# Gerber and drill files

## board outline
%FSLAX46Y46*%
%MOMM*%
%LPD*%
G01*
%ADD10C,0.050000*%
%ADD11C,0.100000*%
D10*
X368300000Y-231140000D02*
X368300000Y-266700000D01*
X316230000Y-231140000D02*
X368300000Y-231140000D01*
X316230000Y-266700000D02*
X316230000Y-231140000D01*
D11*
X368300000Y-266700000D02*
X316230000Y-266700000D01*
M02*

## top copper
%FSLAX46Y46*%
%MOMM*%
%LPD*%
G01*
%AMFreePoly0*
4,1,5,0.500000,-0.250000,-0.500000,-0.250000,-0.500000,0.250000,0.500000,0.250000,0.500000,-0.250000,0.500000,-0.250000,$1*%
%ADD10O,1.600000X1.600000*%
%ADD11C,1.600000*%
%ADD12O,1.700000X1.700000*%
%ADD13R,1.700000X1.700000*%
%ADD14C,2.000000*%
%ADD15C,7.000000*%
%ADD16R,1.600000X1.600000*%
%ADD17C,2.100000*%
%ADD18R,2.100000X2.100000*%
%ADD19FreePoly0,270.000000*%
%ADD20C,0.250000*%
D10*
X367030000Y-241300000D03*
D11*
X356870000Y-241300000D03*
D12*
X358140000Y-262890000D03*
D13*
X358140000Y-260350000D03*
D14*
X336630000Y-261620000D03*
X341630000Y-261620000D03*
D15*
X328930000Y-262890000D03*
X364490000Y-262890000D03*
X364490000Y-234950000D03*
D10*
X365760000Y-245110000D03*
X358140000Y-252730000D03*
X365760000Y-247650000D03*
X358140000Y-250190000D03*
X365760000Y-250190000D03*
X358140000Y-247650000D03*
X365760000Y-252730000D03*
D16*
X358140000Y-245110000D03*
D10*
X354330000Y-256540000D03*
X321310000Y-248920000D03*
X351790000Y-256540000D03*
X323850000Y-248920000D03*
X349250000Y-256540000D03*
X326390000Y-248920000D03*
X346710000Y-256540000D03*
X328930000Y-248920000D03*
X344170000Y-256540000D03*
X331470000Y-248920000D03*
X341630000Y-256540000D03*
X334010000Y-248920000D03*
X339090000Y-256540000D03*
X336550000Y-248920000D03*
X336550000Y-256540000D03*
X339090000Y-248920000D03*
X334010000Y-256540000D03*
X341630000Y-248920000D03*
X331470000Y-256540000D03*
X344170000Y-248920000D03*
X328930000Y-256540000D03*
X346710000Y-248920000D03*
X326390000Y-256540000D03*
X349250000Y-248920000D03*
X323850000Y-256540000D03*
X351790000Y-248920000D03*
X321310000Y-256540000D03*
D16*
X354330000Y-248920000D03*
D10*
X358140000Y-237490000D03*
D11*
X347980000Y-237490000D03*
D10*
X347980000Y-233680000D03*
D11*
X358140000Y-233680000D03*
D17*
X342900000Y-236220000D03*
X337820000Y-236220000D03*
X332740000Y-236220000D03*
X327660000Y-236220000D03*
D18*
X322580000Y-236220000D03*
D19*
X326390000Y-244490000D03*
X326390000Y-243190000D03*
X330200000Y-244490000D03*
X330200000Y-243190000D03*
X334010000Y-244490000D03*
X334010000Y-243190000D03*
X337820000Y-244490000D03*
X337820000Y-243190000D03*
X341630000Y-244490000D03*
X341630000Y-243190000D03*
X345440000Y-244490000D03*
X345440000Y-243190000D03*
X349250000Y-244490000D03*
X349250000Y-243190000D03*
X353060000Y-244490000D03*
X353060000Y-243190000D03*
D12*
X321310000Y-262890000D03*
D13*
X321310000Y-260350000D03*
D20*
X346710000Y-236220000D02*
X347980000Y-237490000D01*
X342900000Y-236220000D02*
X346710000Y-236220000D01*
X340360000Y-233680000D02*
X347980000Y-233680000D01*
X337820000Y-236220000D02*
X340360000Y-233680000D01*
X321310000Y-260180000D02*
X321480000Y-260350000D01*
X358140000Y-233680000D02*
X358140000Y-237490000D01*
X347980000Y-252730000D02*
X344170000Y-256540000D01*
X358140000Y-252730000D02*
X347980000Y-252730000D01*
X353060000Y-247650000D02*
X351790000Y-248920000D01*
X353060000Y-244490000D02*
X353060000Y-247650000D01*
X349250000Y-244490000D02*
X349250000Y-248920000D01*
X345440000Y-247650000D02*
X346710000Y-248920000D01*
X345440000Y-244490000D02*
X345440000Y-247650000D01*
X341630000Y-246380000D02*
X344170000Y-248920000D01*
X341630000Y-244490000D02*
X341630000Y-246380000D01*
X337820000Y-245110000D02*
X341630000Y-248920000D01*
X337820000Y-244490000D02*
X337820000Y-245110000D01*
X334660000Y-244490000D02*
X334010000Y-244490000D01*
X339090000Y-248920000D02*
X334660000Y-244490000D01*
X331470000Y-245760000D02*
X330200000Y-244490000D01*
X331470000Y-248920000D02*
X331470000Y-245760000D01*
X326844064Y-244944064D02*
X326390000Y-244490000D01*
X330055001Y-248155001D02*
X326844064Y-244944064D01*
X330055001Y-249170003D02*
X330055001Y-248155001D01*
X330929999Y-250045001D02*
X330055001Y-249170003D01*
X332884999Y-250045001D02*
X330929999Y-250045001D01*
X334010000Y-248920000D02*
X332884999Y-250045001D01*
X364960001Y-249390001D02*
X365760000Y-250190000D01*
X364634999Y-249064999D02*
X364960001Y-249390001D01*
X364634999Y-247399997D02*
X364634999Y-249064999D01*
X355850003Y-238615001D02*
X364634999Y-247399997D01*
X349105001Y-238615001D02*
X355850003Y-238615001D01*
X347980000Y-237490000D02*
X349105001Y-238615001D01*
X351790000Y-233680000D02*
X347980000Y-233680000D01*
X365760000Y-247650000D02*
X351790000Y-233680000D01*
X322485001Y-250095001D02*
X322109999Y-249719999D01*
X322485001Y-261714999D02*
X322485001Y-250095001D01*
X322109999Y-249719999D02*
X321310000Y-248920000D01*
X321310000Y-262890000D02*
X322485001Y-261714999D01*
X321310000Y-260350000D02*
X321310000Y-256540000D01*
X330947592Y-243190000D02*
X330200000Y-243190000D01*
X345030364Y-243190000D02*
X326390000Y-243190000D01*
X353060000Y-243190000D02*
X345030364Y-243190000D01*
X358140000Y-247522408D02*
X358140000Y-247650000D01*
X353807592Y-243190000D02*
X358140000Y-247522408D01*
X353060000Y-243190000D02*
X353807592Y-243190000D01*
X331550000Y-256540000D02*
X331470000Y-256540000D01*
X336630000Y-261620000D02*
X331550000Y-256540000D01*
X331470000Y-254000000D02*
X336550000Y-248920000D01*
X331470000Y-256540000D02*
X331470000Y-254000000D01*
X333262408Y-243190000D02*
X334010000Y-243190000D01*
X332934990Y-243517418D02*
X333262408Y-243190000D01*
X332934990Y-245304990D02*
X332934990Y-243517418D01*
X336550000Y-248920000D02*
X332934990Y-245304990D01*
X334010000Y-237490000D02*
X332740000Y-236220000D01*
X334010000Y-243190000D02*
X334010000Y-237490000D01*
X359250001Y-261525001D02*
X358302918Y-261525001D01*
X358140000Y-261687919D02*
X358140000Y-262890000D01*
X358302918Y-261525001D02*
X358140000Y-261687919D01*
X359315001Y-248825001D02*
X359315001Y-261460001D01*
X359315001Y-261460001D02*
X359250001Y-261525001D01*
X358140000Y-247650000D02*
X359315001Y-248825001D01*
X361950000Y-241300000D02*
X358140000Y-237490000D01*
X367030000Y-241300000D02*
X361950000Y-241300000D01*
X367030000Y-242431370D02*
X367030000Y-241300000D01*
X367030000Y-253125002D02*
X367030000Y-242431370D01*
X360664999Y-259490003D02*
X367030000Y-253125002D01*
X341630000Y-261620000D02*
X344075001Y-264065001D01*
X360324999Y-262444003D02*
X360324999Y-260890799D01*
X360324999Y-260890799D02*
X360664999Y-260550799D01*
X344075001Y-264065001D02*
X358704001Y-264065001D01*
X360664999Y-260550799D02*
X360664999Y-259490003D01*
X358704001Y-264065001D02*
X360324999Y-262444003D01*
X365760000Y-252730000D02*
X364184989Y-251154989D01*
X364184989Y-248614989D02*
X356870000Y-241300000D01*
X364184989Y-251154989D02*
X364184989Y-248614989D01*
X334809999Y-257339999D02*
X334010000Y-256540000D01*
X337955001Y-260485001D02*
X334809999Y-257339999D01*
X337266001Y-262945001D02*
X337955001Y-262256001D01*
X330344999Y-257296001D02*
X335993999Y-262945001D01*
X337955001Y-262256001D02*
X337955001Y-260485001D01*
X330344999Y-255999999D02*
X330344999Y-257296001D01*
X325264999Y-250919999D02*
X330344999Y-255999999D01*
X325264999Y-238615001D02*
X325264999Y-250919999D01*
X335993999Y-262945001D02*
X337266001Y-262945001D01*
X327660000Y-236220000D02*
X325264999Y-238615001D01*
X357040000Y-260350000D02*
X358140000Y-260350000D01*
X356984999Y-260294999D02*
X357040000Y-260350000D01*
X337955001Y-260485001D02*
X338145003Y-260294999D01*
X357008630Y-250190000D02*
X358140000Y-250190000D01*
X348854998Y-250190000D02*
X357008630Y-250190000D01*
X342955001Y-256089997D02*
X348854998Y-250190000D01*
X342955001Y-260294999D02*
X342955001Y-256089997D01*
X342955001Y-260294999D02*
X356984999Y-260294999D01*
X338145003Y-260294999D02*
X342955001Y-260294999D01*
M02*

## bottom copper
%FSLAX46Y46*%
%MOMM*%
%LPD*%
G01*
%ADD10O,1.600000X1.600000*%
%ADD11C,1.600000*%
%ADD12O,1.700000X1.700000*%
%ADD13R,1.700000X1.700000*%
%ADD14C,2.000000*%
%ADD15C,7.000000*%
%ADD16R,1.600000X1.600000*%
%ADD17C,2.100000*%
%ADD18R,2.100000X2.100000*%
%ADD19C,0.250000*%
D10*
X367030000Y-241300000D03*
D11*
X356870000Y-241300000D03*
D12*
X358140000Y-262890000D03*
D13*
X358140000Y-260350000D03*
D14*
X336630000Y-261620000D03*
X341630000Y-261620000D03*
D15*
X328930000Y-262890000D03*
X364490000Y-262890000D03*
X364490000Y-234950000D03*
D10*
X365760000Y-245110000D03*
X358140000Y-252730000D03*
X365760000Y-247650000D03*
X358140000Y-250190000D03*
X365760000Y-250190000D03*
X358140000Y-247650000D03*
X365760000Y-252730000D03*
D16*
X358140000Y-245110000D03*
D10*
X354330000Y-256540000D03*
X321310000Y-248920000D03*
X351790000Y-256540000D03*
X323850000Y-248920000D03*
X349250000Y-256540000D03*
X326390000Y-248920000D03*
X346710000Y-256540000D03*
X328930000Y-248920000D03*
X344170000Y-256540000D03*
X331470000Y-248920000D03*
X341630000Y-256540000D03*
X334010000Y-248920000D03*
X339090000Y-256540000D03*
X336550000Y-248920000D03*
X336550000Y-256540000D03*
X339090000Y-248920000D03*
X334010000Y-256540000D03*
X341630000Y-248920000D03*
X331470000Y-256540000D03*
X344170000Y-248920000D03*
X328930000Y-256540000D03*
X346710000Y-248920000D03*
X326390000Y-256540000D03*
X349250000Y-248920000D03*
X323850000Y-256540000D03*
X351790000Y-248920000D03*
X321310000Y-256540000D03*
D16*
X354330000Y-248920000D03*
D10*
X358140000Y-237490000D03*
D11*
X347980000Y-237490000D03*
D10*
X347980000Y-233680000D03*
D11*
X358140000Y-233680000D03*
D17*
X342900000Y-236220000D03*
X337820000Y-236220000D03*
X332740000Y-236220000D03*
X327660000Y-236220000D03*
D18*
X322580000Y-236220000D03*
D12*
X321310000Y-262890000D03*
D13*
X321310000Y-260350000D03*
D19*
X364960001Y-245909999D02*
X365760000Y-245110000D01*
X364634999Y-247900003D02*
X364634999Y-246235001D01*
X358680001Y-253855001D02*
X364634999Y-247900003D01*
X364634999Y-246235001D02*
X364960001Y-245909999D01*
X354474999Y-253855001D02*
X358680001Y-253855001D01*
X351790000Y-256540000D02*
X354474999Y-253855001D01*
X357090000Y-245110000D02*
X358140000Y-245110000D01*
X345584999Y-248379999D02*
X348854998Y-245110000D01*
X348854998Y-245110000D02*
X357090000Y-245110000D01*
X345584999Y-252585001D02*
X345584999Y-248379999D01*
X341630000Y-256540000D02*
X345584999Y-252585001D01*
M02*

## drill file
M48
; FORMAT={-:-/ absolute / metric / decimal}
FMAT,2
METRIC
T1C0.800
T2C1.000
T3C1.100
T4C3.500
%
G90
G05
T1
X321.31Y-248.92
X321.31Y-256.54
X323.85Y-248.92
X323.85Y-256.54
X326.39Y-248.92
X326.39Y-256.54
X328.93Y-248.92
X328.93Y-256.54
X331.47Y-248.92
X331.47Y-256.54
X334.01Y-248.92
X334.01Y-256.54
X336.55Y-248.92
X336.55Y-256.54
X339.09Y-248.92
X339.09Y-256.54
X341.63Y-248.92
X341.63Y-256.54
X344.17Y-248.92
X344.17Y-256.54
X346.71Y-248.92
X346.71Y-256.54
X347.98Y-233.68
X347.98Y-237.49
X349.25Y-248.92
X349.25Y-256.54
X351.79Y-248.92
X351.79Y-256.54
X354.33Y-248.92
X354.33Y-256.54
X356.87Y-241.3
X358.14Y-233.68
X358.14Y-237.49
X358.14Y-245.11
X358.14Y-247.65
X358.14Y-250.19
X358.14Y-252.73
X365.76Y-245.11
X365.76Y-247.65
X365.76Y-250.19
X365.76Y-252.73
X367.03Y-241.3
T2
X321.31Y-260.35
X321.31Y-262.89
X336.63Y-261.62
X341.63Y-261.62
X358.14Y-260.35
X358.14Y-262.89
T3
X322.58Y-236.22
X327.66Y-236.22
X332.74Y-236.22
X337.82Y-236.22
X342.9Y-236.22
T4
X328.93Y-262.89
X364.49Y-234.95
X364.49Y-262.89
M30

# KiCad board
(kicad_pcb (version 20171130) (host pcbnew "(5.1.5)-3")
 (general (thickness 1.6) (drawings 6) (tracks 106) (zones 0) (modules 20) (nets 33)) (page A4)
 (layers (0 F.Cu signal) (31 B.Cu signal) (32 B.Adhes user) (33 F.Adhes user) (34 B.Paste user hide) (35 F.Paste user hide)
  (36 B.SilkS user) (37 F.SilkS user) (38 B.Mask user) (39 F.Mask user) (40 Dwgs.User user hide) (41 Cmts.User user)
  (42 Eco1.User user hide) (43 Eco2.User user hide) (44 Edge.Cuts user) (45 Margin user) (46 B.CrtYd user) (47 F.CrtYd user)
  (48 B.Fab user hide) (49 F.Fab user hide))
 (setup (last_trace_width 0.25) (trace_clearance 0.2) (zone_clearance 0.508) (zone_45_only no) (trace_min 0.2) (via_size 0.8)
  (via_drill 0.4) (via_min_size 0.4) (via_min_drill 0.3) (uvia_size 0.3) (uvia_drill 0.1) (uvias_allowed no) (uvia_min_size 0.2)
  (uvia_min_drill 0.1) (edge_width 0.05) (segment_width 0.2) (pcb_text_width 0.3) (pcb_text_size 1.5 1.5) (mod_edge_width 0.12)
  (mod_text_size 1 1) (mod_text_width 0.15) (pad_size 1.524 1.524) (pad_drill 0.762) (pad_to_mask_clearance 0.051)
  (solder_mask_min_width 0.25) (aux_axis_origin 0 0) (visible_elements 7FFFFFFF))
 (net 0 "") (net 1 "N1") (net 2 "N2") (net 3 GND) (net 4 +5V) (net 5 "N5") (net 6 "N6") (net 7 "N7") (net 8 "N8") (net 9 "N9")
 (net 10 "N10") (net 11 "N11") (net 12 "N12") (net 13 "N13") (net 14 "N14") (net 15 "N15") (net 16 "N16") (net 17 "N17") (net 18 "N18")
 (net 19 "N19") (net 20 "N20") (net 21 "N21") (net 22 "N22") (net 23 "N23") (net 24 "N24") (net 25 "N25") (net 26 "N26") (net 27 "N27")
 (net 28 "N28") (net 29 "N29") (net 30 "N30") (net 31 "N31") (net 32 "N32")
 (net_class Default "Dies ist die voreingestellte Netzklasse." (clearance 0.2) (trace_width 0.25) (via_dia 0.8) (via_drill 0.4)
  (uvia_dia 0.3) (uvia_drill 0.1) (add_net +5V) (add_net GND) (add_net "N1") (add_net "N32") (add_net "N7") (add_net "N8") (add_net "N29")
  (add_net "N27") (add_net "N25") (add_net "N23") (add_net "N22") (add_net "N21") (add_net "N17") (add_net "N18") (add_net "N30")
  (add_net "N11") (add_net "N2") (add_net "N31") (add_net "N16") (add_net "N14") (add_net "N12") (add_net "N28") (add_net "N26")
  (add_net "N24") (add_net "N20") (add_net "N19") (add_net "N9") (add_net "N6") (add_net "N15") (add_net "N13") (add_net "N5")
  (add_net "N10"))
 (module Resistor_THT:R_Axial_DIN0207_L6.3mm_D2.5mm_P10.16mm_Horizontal (layer F.Cu) (at 356.87 241.3)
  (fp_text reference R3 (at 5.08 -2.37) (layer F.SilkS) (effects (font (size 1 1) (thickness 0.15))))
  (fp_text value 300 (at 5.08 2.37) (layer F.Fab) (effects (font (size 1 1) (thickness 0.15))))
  (pad 2 thru_hole oval (at 10.16 0) (size 1.6 1.6) (drill 0.8) (layers *.Cu *.Mask) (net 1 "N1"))
  (pad 1 thru_hole circle (at 0 0) (size 1.6 1.6) (drill 0.8) (layers *.Cu *.Mask) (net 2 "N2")))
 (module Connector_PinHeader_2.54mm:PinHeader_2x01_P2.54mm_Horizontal (layer F.Cu) (at 358.14 260.35 270)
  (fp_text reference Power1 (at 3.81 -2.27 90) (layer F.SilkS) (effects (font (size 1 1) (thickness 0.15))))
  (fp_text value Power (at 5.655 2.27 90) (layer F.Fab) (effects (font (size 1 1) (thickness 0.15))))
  (pad 2 thru_hole oval (at 2.54 0 270) (size 1.7 1.7) (drill 1) (layers *.Cu *.Mask) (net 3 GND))
  (pad 1 thru_hole rect (at 0 0 270) (size 1.7 1.7) (drill 1) (layers *.Cu *.Mask) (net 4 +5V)))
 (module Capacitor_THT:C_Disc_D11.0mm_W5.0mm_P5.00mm (layer F.Cu) (at 341.63 261.62 180)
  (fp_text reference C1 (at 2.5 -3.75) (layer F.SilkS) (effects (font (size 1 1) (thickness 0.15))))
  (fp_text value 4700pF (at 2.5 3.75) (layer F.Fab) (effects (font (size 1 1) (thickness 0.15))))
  (pad 2 thru_hole circle (at 5 0 180) (size 2 2) (drill 1) (layers *.Cu *.Mask) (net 3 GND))
  (pad 1 thru_hole circle (at 0 0 180) (size 2 2) (drill 1) (layers *.Cu *.Mask) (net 1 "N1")))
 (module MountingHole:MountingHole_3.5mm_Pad (layer F.Cu) (at 328.93 262.89) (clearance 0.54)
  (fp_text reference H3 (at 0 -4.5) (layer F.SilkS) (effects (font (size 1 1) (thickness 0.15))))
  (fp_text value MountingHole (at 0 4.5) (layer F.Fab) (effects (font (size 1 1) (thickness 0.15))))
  (pad 1 thru_hole circle (at 0 0) (size 7 7) (drill 3.5) (layers *.Cu *.Mask)))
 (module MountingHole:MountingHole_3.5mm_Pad (layer F.Cu) (at 364.49 262.89) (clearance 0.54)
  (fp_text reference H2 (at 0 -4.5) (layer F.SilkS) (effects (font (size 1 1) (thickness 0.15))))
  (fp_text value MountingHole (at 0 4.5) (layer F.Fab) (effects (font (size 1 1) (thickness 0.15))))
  (pad 1 thru_hole circle (at 0 0) (size 7 7) (drill 3.5) (layers *.Cu *.Mask)))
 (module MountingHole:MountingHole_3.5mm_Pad (layer F.Cu) (at 364.49 234.95 180) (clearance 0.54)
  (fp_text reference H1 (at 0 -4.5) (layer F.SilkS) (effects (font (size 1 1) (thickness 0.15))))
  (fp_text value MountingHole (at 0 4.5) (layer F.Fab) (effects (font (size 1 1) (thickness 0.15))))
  (pad 1 thru_hole circle (at 0 0 180) (size 7 7) (drill 3.5) (layers *.Cu *.Mask)))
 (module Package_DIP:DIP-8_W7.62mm (layer F.Cu) (at 358.14 245.11)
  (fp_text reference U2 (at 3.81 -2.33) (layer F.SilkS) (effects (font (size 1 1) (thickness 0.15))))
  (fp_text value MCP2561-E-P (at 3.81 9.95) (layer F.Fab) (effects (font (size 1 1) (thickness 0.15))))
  (pad 8 thru_hole oval (at 7.62 0) (size 1.6 1.6) (drill 0.8) (layers *.Cu *.Mask) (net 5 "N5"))
  (pad 4 thru_hole oval (at 0 7.62) (size 1.6 1.6) (drill 0.8) (layers *.Cu *.Mask) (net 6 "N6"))
  (pad 7 thru_hole oval (at 7.62 2.54) (size 1.6 1.6) (drill 0.8) (layers *.Cu *.Mask) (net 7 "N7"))
  (pad 3 thru_hole oval (at 0 5.08) (size 1.6 1.6) (drill 0.8) (layers *.Cu *.Mask) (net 4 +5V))
  (pad 6 thru_hole oval (at 7.62 5.08) (size 1.6 1.6) (drill 0.8) (layers *.Cu *.Mask) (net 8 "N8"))
  (pad 2 thru_hole oval (at 0 2.54) (size 1.6 1.6) (drill 0.8) (layers *.Cu *.Mask) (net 3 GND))
  (pad 5 thru_hole oval (at 7.62 7.62) (size 1.6 1.6) (drill 0.8) (layers *.Cu *.Mask) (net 2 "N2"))
  (pad 1 thru_hole rect (at 0 0) (size 1.6 1.6) (drill 0.8) (layers *.Cu *.Mask) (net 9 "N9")))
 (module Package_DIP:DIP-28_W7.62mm (layer F.Cu) (at 354.33 248.92 270)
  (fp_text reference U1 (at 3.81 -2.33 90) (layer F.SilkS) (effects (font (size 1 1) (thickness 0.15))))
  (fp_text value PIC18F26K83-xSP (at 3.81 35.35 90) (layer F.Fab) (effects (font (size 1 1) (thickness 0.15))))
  (pad 28 thru_hole oval (at 7.62 0 270) (size 1.6 1.6) (drill 0.8) (layers *.Cu *.Mask) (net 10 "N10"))
  (pad 14 thru_hole oval (at 0 33.02 270) (size 1.6 1.6) (drill 0.8) (layers *.Cu *.Mask) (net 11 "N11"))
  (pad 27 thru_hole oval (at 7.62 2.54 270) (size 1.6 1.6) (drill 0.8) (layers *.Cu *.Mask) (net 5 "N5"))
  (pad 13 thru_hole oval (at 0 30.48 270) (size 1.6 1.6) (drill 0.8) (layers *.Cu *.Mask) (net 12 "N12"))
  (pad 26 thru_hole oval (at 7.62 5.08 270) (size 1.6 1.6) (drill 0.8) (layers *.Cu *.Mask) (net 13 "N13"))
  (pad 12 thru_hole oval (at 0 27.94 270) (size 1.6 1.6) (drill 0.8) (layers *.Cu *.Mask) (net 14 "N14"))
  (pad 25 thru_hole oval (at 7.62 7.62 270) (size 1.6 1.6) (drill 0.8) (layers *.Cu *.Mask) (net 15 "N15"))
  (pad 11 thru_hole oval (at 0 25.4 270) (size 1.6 1.6) (drill 0.8) (layers *.Cu *.Mask) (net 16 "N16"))
  (pad 24 thru_hole oval (at 7.62 10.16 270) (size 1.6 1.6) (drill 0.8) (layers *.Cu *.Mask) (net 6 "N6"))
  (pad 10 thru_hole oval (at 0 22.86 270) (size 1.6 1.6) (drill 0.8) (layers *.Cu *.Mask) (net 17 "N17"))
  (pad 23 thru_hole oval (at 7.62 12.7 270) (size 1.6 1.6) (drill 0.8) (layers *.Cu *.Mask) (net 9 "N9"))
  (pad 9 thru_hole oval (at 0 20.32 270) (size 1.6 1.6) (drill 0.8) (layers *.Cu *.Mask) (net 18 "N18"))
  (pad 22 thru_hole oval (at 7.62 15.24 270) (size 1.6 1.6) (drill 0.8) (layers *.Cu *.Mask) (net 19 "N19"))
  (pad 8 thru_hole oval (at 0 17.78 270) (size 1.6 1.6) (drill 0.8) (layers *.Cu *.Mask) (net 3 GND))
  (pad 21 thru_hole oval (at 7.62 17.78 270) (size 1.6 1.6) (drill 0.8) (layers *.Cu *.Mask) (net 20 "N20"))
  (pad 7 thru_hole oval (at 0 15.24 270) (size 1.6 1.6) (drill 0.8) (layers *.Cu *.Mask) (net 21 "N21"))
  (pad 20 thru_hole oval (at 7.62 20.32 270) (size 1.6 1.6) (drill 0.8) (layers *.Cu *.Mask) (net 4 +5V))
  (pad 6 thru_hole oval (at 0 12.7 270) (size 1.6 1.6) (drill 0.8) (layers *.Cu *.Mask) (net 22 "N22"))
  (pad 19 thru_hole oval (at 7.62 22.86 270) (size 1.6 1.6) (drill 0.8) (layers *.Cu *.Mask) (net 3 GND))
  (pad 5 thru_hole oval (at 0 10.16 270) (size 1.6 1.6) (drill 0.8) (layers *.Cu *.Mask) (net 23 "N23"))
  (pad 18 thru_hole oval (at 7.62 25.4 270) (size 1.6 1.6) (drill 0.8) (layers *.Cu *.Mask) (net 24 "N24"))
  (pad 4 thru_hole oval (at 0 7.62 270) (size 1.6 1.6) (drill 0.8) (layers *.Cu *.Mask) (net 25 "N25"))
  (pad 17 thru_hole oval (at 7.62 27.94 270) (size 1.6 1.6) (drill 0.8) (layers *.Cu *.Mask) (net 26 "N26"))
  (pad 3 thru_hole oval (at 0 5.08 270) (size 1.6 1.6) (drill 0.8) (layers *.Cu *.Mask) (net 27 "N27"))
  (pad 16 thru_hole oval (at 7.62 30.48 270) (size 1.6 1.6) (drill 0.8) (layers *.Cu *.Mask) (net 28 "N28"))
  (pad 2 thru_hole oval (at 0 2.54 270) (size 1.6 1.6) (drill 0.8) (layers *.Cu *.Mask) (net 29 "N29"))
  (pad 15 thru_hole oval (at 7.62 33.02 270) (size 1.6 1.6) (drill 0.8) (layers *.Cu *.Mask) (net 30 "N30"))
  (pad 1 thru_hole rect (at 0 0 270) (size 1.6 1.6) (drill 0.8) (layers *.Cu *.Mask) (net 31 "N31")))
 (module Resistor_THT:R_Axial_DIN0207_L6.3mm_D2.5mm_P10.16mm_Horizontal (layer F.Cu) (at 347.98 237.49)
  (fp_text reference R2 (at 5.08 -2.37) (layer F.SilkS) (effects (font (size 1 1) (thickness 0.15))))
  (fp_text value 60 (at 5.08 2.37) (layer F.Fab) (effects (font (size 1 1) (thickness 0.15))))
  (pad 2 thru_hole oval (at 10.16 0) (size 1.6 1.6) (drill 0.8) (layers *.Cu *.Mask) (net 1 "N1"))
  (pad 1 thru_hole circle (at 0 0) (size 1.6 1.6) (drill 0.8) (layers *.Cu *.Mask) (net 8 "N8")))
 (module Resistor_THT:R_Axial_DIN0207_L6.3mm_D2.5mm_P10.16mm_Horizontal (layer F.Cu) (at 358.14 233.68 180)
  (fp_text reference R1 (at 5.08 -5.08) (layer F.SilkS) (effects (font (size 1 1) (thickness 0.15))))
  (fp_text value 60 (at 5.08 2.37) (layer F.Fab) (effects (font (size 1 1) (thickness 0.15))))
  (pad 2 thru_hole oval (at 10.16 0 180) (size 1.6 1.6) (drill 0.8) (layers *.Cu *.Mask) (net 7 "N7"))
  (pad 1 thru_hole circle (at 0 0 180) (size 1.6 1.6) (drill 0.8) (layers *.Cu *.Mask) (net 1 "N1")))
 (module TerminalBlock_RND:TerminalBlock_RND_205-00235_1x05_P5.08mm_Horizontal (layer F.Cu) (at 322.58 236.22)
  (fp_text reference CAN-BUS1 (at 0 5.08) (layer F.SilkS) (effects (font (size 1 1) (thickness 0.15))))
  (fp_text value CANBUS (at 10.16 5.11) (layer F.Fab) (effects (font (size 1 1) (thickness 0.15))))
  (pad 5 thru_hole circle (at 20.32 0) (size 2.1 2.1) (drill 1.1) (layers *.Cu *.Mask) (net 8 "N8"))
  (pad 4 thru_hole circle (at 15.24 0) (size 2.1 2.1) (drill 1.1) (layers *.Cu *.Mask) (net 7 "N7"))
  (pad 3 thru_hole circle (at 10.16 0) (size 2.1 2.1) (drill 1.1) (layers *.Cu *.Mask) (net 3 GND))
  (pad 2 thru_hole circle (at 5.08 0) (size 2.1 2.1) (drill 1.1) (layers *.Cu *.Mask) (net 4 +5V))
  (pad 1 thru_hole rect (at 0 0) (size 2.1 2.1) (drill 1.1) (layers *.Cu *.Mask) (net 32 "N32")))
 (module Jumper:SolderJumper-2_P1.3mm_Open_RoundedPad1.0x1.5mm (layer F.Cu) (at 326.39 243.84 270)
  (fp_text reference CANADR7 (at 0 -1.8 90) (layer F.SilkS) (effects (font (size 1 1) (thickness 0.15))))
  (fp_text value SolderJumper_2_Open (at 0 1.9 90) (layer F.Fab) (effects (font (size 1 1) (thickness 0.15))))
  (pad 2 smd custom (at 0.65 0 270) (size 1 0.5) (layers F.Cu F.Mask) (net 18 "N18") (zone_connect 2)
   (options (clearance outline) (anchor rect)) (primitives))
  (pad 1 smd custom (at -0.65 0 270) (size 1 0.5) (layers F.Cu F.Mask) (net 3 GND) (zone_connect 2)
   (options (clearance outline) (anchor rect)) (primitives)))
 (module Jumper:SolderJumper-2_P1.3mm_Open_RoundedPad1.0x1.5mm (layer F.Cu) (at 330.2 243.84 270)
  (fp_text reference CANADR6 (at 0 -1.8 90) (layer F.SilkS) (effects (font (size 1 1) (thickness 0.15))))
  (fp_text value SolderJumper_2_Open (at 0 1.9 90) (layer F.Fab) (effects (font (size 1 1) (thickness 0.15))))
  (pad 2 smd custom (at 0.65 0 270) (size 1 0.5) (layers F.Cu F.Mask) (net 17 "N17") (zone_connect 2)
   (options (clearance outline) (anchor rect)) (primitives))
  (pad 1 smd custom (at -0.65 0 270) (size 1 0.5) (layers F.Cu F.Mask) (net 3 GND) (zone_connect 2)
   (options (clearance outline) (anchor rect)) (primitives)))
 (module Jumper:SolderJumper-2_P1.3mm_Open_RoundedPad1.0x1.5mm (layer F.Cu) (at 334.01 243.84 270)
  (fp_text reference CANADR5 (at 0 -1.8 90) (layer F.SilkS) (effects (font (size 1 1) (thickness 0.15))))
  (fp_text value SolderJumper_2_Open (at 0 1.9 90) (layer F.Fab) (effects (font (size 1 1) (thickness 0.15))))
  (pad 2 smd custom (at 0.65 0 270) (size 1 0.5) (layers F.Cu F.Mask) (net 21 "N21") (zone_connect 2)
   (options (clearance outline) (anchor rect)) (primitives))
  (pad 1 smd custom (at -0.65 0 270) (size 1 0.5) (layers F.Cu F.Mask) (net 3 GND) (zone_connect 2)
   (options (clearance outline) (anchor rect)) (primitives)))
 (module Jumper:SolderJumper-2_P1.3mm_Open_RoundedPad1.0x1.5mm (layer F.Cu) (at 337.82 243.84 270)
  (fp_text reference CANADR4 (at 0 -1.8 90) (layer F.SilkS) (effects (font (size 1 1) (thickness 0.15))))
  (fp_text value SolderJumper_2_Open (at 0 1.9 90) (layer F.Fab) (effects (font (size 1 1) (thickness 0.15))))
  (pad 2 smd custom (at 0.65 0 270) (size 1 0.5) (layers F.Cu F.Mask) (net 22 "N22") (zone_connect 2)
   (options (clearance outline) (anchor rect)) (primitives))
  (pad 1 smd custom (at -0.65 0 270) (size 1 0.5) (layers F.Cu F.Mask) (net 3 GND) (zone_connect 2)
   (options (clearance outline) (anchor rect)) (primitives)))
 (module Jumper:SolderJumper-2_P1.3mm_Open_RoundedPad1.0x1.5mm (layer F.Cu) (at 341.63 243.84 270)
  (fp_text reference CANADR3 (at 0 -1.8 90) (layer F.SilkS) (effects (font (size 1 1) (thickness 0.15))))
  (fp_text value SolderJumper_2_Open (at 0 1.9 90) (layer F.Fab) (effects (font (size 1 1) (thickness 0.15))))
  (pad 2 smd custom (at 0.65 0 270) (size 1 0.5) (layers F.Cu F.Mask) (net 23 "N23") (zone_connect 2)
   (options (clearance outline) (anchor rect)) (primitives))
  (pad 1 smd custom (at -0.65 0 270) (size 1 0.5) (layers F.Cu F.Mask) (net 3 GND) (zone_connect 2)
   (options (clearance outline) (anchor rect)) (primitives)))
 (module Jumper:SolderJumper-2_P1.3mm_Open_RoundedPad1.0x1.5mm (layer F.Cu) (at 345.44 243.84 270)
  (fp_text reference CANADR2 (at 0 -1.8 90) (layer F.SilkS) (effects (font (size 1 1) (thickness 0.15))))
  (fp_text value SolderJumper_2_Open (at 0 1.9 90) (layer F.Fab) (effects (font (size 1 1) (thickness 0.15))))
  (pad 2 smd custom (at 0.65 0 270) (size 1 0.5) (layers F.Cu F.Mask) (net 25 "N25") (zone_connect 2)
   (options (clearance outline) (anchor rect)) (primitives))
  (pad 1 smd custom (at -0.65 0 270) (size 1 0.5) (layers F.Cu F.Mask) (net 3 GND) (zone_connect 2)
   (options (clearance outline) (anchor rect)) (primitives)))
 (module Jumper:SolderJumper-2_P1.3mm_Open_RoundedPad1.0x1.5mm (layer F.Cu) (at 349.25 243.84 270)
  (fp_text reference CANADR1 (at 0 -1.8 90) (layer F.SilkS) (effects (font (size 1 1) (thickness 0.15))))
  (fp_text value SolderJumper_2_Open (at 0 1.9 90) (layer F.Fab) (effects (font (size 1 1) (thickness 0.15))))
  (pad 2 smd custom (at 0.65 0 270) (size 1 0.5) (layers F.Cu F.Mask) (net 27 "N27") (zone_connect 2)
   (options (clearance outline) (anchor rect)) (primitives))
  (pad 1 smd custom (at -0.65 0 270) (size 1 0.5) (layers F.Cu F.Mask) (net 3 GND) (zone_connect 2)
   (options (clearance outline) (anchor rect)) (primitives)))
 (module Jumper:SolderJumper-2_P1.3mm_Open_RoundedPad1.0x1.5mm (layer F.Cu) (at 353.06 243.84 270)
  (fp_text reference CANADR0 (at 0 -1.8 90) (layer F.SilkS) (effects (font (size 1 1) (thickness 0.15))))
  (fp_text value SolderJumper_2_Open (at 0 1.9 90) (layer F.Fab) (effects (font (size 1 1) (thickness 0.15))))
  (pad 2 smd custom (at 0.65 0 270) (size 1 0.5) (layers F.Cu F.Mask) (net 29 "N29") (zone_connect 2)
   (options (clearance outline) (anchor rect)) (primitives))
  (pad 1 smd custom (at -0.65 0 270) (size 1 0.5) (layers F.Cu F.Mask) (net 3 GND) (zone_connect 2)
   (options (clearance outline) (anchor rect)) (primitives)))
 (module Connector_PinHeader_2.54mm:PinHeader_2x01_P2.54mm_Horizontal (layer F.Cu) (at 321.31 260.35 270)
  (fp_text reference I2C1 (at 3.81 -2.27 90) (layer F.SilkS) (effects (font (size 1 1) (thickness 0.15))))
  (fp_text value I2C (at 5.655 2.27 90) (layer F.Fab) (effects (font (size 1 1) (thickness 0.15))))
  (pad 2 thru_hole oval (at 2.54 0 270) (size 1.7 1.7) (drill 1) (layers *.Cu *.Mask) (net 11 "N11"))
  (pad 1 thru_hole rect (at 0 0 270) (size 1.7 1.7) (drill 1) (layers *.Cu *.Mask) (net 30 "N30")))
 (gr_line (start 368.3 231.14) (end 368.3 266.7) (layer Edge.Cuts) (width 0.05))
 (gr_line (start 316.23 231.14) (end 368.3 231.14) (layer Edge.Cuts) (width 0.05))
 (gr_line (start 316.23 266.7) (end 316.23 231.14) (layer Edge.Cuts) (width 0.05))
 (gr_line (start 368.3 266.7) (end 316.23 266.7) (layer Edge.Cuts) (width 0.1))
 (segment (start 364.960001 245.909999) (end 365.76 245.11) (width 0.25) (layer B.Cu) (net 5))
 (segment (start 364.634999 247.900003) (end 364.634999 246.235001) (width 0.25) (layer B.Cu) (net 5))
 (segment (start 358.680001 253.855001) (end 364.634999 247.900003) (width 0.25) (layer B.Cu) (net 5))
 (segment (start 364.634999 246.235001) (end 364.960001 245.909999) (width 0.25) (layer B.Cu) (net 5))
 (segment (start 354.474999 253.855001) (end 358.680001 253.855001) (width 0.25) (layer B.Cu) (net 5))
 (segment (start 351.79 256.54) (end 354.474999 253.855001) (width 0.25) (layer B.Cu) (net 5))
 (segment (start 346.71 236.22) (end 347.98 237.49) (width 0.25) (layer F.Cu) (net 8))
 (segment (start 342.9 236.22) (end 346.71 236.22) (width 0.25) (layer F.Cu) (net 8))
 (segment (start 340.36 233.68) (end 347.98 233.68) (width 0.25) (layer F.Cu) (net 7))
 (segment (start 337.82 236.22) (end 340.36 233.68) (width 0.25) (layer F.Cu) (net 7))
 (segment (start 321.31 260.18) (end 321.48 260.35) (width 0.25) (layer F.Cu) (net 30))
 (segment (start 358.14 233.68) (end 358.14 237.49) (width 0.25) (layer F.Cu) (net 1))
 (segment (start 347.98 252.73) (end 344.17 256.54) (width 0.25) (layer F.Cu) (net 6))
 (segment (start 358.14 252.73) (end 347.98 252.73) (width 0.25) (layer F.Cu) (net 6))
 (segment (start 357.09 245.11) (end 358.14 245.11) (width 0.25) (layer B.Cu) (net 9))
 (segment (start 345.584999 248.379999) (end 348.854998 245.11) (width 0.25) (layer B.Cu) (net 9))
 (segment (start 348.854998 245.11) (end 357.09 245.11) (width 0.25) (layer B.Cu) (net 9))
 (segment (start 345.584999 252.585001) (end 345.584999 248.379999) (width 0.25) (layer B.Cu) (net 9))
 (segment (start 341.63 256.54) (end 345.584999 252.585001) (width 0.25) (layer B.Cu) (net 9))
 (segment (start 353.06 247.65) (end 351.79 248.92) (width 0.25) (layer F.Cu) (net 29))
 (segment (start 353.06 244.49) (end 353.06 247.65) (width 0.25) (layer F.Cu) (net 29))
 (segment (start 349.25 244.49) (end 349.25 248.92) (width 0.25) (layer F.Cu) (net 27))
 (segment (start 345.44 247.65) (end 346.71 248.92) (width 0.25) (layer F.Cu) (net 25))
 (segment (start 345.44 244.49) (end 345.44 247.65) (width 0.25) (layer F.Cu) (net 25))
 (segment (start 341.63 246.38) (end 344.17 248.92) (width 0.25) (layer F.Cu) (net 23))
 (segment (start 341.63 244.49) (end 341.63 246.38) (width 0.25) (layer F.Cu) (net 23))
 (segment (start 337.82 245.11) (end 341.63 248.92) (width 0.25) (layer F.Cu) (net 22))
 (segment (start 337.82 244.49) (end 337.82 245.11) (width 0.25) (layer F.Cu) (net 22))
 (segment (start 334.66 244.49) (end 334.01 244.49) (width 0.25) (layer F.Cu) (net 21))
 (segment (start 339.09 248.92) (end 334.66 244.49) (width 0.25) (layer F.Cu) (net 21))
 (segment (start 331.47 245.76) (end 330.2 244.49) (width 0.25) (layer F.Cu) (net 17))
 (segment (start 331.47 248.92) (end 331.47 245.76) (width 0.25) (layer F.Cu) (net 17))
 (segment (start 326.844064 244.944064) (end 326.39 244.49) (width 0.25) (layer F.Cu) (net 18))
 (segment (start 330.055001 248.155001) (end 326.844064 244.944064) (width 0.25) (layer F.Cu) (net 18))
 (segment (start 330.055001 249.170003) (end 330.055001 248.155001) (width 0.25) (layer F.Cu) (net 18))
 (segment (start 330.929999 250.045001) (end 330.055001 249.170003) (width 0.25) (layer F.Cu) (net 18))
 (segment (start 332.884999 250.045001) (end 330.929999 250.045001) (width 0.25) (layer F.Cu) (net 18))
 (segment (start 334.01 248.92) (end 332.884999 250.045001) (width 0.25) (layer F.Cu) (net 18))
 (segment (start 364.960001 249.390001) (end 365.76 250.19) (width 0.25) (layer F.Cu) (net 8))
 (segment (start 364.634999 249.064999) (end 364.960001 249.390001) (width 0.25) (layer F.Cu) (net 8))
 (segment (start 364.634999 247.399997) (end 364.634999 249.064999) (width 0.25) (layer F.Cu) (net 8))
 (segment (start 355.850003 238.615001) (end 364.634999 247.399997) (width 0.25) (layer F.Cu) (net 8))
 (segment (start 349.105001 238.615001) (end 355.850003 238.615001) (width 0.25) (layer F.Cu) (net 8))
 (segment (start 347.98 237.49) (end 349.105001 238.615001) (width 0.25) (layer F.Cu) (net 8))
 (segment (start 351.79 233.68) (end 347.98 233.68) (width 0.25) (layer F.Cu) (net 7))
 (segment (start 365.76 247.65) (end 351.79 233.68) (width 0.25) (layer F.Cu) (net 7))
 (segment (start 322.485001 250.095001) (end 322.109999 249.719999) (width 0.25) (layer F.Cu) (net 11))
 (segment (start 322.485001 261.714999) (end 322.485001 250.095001) (width 0.25) (layer F.Cu) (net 11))
 (segment (start 322.109999 249.719999) (end 321.31 248.92) (width 0.25) (layer F.Cu) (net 11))
 (segment (start 321.31 262.89) (end 322.485001 261.714999) (width 0.25) (layer F.Cu) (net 11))
 (segment (start 321.31 260.35) (end 321.31 256.54) (width 0.25) (layer F.Cu) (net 30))
 (segment (start 330.947592 243.19) (end 330.2 243.19) (width 0.25) (layer F.Cu) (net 3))
 (segment (start 345.030364 243.19) (end 326.39 243.19) (width 0.25) (layer F.Cu) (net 3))
 (segment (start 353.06 243.19) (end 345.030364 243.19) (width 0.25) (layer F.Cu) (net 3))
 (segment (start 358.14 247.522408) (end 358.14 247.65) (width 0.25) (layer F.Cu) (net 3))
 (segment (start 353.807592 243.19) (end 358.14 247.522408) (width 0.25) (layer F.Cu) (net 3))
 (segment (start 353.06 243.19) (end 353.807592 243.19) (width 0.25) (layer F.Cu) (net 3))
 (segment (start 331.55 256.54) (end 331.47 256.54) (width 0.25) (layer F.Cu) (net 3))
 (segment (start 336.63 261.62) (end 331.55 256.54) (width 0.25) (layer F.Cu) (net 3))
 (segment (start 331.47 254) (end 336.55 248.92) (width 0.25) (layer F.Cu) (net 3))
 (segment (start 331.47 256.54) (end 331.47 254) (width 0.25) (layer F.Cu) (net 3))
 (segment (start 333.262408 243.19) (end 334.01 243.19) (width 0.25) (layer F.Cu) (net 3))
 (segment (start 332.93499 243.517418) (end 333.262408 243.19) (width 0.25) (layer F.Cu) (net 3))
 (segment (start 332.93499 245.30499) (end 332.93499 243.517418) (width 0.25) (layer F.Cu) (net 3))
 (segment (start 336.55 248.92) (end 332.93499 245.30499) (width 0.25) (layer F.Cu) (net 3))
 (segment (start 334.01 237.49) (end 332.74 236.22) (width 0.25) (layer F.Cu) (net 3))
 (segment (start 334.01 243.19) (end 334.01 237.49) (width 0.25) (layer F.Cu) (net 3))
 (segment (start 359.250001 261.525001) (end 358.302918 261.525001) (width 0.25) (layer F.Cu) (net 3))
 (segment (start 358.14 261.687919) (end 358.14 262.89) (width 0.25) (layer F.Cu) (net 3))
 (segment (start 358.302918 261.525001) (end 358.14 261.687919) (width 0.25) (layer F.Cu) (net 3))
 (segment (start 359.315001 248.825001) (end 359.315001 261.460001) (width 0.25) (layer F.Cu) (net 3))
 (segment (start 359.315001 261.460001) (end 359.250001 261.525001) (width 0.25) (layer F.Cu) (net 3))
 (segment (start 358.14 247.65) (end 359.315001 248.825001) (width 0.25) (layer F.Cu) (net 3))
 (segment (start 361.95 241.3) (end 358.14 237.49) (width 0.25) (layer F.Cu) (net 1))
 (segment (start 367.03 241.3) (end 361.95 241.3) (width 0.25) (layer F.Cu) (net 1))
 (segment (start 367.03 242.43137) (end 367.03 241.3) (width 0.25) (layer F.Cu) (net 1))
 (segment (start 367.03 253.125002) (end 367.03 242.43137) (width 0.25) (layer F.Cu) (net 1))
 (segment (start 360.664999 259.490003) (end 367.03 253.125002) (width 0.25) (layer F.Cu) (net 1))
 (segment (start 341.63 261.62) (end 344.075001 264.065001) (width 0.25) (layer F.Cu) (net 1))
 (segment (start 360.324999 262.444003) (end 360.324999 260.890799) (width 0.25) (layer F.Cu) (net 1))
 (segment (start 360.324999 260.890799) (end 360.664999 260.550799) (width 0.25) (layer F.Cu) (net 1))
 (segment (start 344.075001 264.065001) (end 358.704001 264.065001) (width 0.25) (layer F.Cu) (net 1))
 (segment (start 360.664999 260.550799) (end 360.664999 259.490003) (width 0.25) (layer F.Cu) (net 1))
 (segment (start 358.704001 264.065001) (end 360.324999 262.444003) (width 0.25) (layer F.Cu) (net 1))
 (segment (start 365.76 252.73) (end 364.184989 251.154989) (width 0.25) (layer F.Cu) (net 2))
 (segment (start 364.184989 248.614989) (end 356.87 241.3) (width 0.25) (layer F.Cu) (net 2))
 (segment (start 364.184989 251.154989) (end 364.184989 248.614989) (width 0.25) (layer F.Cu) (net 2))
 (segment (start 334.809999 257.339999) (end 334.01 256.54) (width 0.25) (layer F.Cu) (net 4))
 (segment (start 337.955001 260.485001) (end 334.809999 257.339999) (width 0.25) (layer F.Cu) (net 4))
 (segment (start 337.266001 262.945001) (end 337.955001 262.256001) (width 0.25) (layer F.Cu) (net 4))
 (segment (start 330.344999 257.296001) (end 335.993999 262.945001) (width 0.25) (layer F.Cu) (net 4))
 (segment (start 337.955001 262.256001) (end 337.955001 260.485001) (width 0.25) (layer F.Cu) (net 4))
 (segment (start 330.344999 255.999999) (end 330.344999 257.296001) (width 0.25) (layer F.Cu) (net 4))
 (segment (start 325.264999 250.919999) (end 330.344999 255.999999) (width 0.25) (layer F.Cu) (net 4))
 (segment (start 325.264999 238.615001) (end 325.264999 250.919999) (width 0.25) (layer F.Cu) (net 4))
 (segment (start 335.993999 262.945001) (end 337.266001 262.945001) (width 0.25) (layer F.Cu) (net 4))
 (segment (start 327.66 236.22) (end 325.264999 238.615001) (width 0.25) (layer F.Cu) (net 4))
 (segment (start 357.04 260.35) (end 358.14 260.35) (width 0.25) (layer F.Cu) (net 4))
 (segment (start 356.984999 260.294999) (end 357.04 260.35) (width 0.25) (layer F.Cu) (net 4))
 (segment (start 337.955001 260.485001) (end 338.145003 260.294999) (width 0.25) (layer F.Cu) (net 4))
 (segment (start 357.00863 250.19) (end 358.14 250.19) (width 0.25) (layer F.Cu) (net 4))
 (segment (start 348.854998 250.19) (end 357.00863 250.19) (width 0.25) (layer F.Cu) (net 4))
 (segment (start 342.955001 256.089997) (end 348.854998 250.19) (width 0.25) (layer F.Cu) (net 4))
 (segment (start 342.955001 260.294999) (end 342.955001 256.089997) (width 0.25) (layer F.Cu) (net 4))
 (segment (start 342.955001 260.294999) (end 356.984999 260.294999) (width 0.25) (layer F.Cu) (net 4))
 (segment (start 338.145003 260.294999) (end 342.955001 260.294999) (width 0.25) (layer F.Cu) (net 4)))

